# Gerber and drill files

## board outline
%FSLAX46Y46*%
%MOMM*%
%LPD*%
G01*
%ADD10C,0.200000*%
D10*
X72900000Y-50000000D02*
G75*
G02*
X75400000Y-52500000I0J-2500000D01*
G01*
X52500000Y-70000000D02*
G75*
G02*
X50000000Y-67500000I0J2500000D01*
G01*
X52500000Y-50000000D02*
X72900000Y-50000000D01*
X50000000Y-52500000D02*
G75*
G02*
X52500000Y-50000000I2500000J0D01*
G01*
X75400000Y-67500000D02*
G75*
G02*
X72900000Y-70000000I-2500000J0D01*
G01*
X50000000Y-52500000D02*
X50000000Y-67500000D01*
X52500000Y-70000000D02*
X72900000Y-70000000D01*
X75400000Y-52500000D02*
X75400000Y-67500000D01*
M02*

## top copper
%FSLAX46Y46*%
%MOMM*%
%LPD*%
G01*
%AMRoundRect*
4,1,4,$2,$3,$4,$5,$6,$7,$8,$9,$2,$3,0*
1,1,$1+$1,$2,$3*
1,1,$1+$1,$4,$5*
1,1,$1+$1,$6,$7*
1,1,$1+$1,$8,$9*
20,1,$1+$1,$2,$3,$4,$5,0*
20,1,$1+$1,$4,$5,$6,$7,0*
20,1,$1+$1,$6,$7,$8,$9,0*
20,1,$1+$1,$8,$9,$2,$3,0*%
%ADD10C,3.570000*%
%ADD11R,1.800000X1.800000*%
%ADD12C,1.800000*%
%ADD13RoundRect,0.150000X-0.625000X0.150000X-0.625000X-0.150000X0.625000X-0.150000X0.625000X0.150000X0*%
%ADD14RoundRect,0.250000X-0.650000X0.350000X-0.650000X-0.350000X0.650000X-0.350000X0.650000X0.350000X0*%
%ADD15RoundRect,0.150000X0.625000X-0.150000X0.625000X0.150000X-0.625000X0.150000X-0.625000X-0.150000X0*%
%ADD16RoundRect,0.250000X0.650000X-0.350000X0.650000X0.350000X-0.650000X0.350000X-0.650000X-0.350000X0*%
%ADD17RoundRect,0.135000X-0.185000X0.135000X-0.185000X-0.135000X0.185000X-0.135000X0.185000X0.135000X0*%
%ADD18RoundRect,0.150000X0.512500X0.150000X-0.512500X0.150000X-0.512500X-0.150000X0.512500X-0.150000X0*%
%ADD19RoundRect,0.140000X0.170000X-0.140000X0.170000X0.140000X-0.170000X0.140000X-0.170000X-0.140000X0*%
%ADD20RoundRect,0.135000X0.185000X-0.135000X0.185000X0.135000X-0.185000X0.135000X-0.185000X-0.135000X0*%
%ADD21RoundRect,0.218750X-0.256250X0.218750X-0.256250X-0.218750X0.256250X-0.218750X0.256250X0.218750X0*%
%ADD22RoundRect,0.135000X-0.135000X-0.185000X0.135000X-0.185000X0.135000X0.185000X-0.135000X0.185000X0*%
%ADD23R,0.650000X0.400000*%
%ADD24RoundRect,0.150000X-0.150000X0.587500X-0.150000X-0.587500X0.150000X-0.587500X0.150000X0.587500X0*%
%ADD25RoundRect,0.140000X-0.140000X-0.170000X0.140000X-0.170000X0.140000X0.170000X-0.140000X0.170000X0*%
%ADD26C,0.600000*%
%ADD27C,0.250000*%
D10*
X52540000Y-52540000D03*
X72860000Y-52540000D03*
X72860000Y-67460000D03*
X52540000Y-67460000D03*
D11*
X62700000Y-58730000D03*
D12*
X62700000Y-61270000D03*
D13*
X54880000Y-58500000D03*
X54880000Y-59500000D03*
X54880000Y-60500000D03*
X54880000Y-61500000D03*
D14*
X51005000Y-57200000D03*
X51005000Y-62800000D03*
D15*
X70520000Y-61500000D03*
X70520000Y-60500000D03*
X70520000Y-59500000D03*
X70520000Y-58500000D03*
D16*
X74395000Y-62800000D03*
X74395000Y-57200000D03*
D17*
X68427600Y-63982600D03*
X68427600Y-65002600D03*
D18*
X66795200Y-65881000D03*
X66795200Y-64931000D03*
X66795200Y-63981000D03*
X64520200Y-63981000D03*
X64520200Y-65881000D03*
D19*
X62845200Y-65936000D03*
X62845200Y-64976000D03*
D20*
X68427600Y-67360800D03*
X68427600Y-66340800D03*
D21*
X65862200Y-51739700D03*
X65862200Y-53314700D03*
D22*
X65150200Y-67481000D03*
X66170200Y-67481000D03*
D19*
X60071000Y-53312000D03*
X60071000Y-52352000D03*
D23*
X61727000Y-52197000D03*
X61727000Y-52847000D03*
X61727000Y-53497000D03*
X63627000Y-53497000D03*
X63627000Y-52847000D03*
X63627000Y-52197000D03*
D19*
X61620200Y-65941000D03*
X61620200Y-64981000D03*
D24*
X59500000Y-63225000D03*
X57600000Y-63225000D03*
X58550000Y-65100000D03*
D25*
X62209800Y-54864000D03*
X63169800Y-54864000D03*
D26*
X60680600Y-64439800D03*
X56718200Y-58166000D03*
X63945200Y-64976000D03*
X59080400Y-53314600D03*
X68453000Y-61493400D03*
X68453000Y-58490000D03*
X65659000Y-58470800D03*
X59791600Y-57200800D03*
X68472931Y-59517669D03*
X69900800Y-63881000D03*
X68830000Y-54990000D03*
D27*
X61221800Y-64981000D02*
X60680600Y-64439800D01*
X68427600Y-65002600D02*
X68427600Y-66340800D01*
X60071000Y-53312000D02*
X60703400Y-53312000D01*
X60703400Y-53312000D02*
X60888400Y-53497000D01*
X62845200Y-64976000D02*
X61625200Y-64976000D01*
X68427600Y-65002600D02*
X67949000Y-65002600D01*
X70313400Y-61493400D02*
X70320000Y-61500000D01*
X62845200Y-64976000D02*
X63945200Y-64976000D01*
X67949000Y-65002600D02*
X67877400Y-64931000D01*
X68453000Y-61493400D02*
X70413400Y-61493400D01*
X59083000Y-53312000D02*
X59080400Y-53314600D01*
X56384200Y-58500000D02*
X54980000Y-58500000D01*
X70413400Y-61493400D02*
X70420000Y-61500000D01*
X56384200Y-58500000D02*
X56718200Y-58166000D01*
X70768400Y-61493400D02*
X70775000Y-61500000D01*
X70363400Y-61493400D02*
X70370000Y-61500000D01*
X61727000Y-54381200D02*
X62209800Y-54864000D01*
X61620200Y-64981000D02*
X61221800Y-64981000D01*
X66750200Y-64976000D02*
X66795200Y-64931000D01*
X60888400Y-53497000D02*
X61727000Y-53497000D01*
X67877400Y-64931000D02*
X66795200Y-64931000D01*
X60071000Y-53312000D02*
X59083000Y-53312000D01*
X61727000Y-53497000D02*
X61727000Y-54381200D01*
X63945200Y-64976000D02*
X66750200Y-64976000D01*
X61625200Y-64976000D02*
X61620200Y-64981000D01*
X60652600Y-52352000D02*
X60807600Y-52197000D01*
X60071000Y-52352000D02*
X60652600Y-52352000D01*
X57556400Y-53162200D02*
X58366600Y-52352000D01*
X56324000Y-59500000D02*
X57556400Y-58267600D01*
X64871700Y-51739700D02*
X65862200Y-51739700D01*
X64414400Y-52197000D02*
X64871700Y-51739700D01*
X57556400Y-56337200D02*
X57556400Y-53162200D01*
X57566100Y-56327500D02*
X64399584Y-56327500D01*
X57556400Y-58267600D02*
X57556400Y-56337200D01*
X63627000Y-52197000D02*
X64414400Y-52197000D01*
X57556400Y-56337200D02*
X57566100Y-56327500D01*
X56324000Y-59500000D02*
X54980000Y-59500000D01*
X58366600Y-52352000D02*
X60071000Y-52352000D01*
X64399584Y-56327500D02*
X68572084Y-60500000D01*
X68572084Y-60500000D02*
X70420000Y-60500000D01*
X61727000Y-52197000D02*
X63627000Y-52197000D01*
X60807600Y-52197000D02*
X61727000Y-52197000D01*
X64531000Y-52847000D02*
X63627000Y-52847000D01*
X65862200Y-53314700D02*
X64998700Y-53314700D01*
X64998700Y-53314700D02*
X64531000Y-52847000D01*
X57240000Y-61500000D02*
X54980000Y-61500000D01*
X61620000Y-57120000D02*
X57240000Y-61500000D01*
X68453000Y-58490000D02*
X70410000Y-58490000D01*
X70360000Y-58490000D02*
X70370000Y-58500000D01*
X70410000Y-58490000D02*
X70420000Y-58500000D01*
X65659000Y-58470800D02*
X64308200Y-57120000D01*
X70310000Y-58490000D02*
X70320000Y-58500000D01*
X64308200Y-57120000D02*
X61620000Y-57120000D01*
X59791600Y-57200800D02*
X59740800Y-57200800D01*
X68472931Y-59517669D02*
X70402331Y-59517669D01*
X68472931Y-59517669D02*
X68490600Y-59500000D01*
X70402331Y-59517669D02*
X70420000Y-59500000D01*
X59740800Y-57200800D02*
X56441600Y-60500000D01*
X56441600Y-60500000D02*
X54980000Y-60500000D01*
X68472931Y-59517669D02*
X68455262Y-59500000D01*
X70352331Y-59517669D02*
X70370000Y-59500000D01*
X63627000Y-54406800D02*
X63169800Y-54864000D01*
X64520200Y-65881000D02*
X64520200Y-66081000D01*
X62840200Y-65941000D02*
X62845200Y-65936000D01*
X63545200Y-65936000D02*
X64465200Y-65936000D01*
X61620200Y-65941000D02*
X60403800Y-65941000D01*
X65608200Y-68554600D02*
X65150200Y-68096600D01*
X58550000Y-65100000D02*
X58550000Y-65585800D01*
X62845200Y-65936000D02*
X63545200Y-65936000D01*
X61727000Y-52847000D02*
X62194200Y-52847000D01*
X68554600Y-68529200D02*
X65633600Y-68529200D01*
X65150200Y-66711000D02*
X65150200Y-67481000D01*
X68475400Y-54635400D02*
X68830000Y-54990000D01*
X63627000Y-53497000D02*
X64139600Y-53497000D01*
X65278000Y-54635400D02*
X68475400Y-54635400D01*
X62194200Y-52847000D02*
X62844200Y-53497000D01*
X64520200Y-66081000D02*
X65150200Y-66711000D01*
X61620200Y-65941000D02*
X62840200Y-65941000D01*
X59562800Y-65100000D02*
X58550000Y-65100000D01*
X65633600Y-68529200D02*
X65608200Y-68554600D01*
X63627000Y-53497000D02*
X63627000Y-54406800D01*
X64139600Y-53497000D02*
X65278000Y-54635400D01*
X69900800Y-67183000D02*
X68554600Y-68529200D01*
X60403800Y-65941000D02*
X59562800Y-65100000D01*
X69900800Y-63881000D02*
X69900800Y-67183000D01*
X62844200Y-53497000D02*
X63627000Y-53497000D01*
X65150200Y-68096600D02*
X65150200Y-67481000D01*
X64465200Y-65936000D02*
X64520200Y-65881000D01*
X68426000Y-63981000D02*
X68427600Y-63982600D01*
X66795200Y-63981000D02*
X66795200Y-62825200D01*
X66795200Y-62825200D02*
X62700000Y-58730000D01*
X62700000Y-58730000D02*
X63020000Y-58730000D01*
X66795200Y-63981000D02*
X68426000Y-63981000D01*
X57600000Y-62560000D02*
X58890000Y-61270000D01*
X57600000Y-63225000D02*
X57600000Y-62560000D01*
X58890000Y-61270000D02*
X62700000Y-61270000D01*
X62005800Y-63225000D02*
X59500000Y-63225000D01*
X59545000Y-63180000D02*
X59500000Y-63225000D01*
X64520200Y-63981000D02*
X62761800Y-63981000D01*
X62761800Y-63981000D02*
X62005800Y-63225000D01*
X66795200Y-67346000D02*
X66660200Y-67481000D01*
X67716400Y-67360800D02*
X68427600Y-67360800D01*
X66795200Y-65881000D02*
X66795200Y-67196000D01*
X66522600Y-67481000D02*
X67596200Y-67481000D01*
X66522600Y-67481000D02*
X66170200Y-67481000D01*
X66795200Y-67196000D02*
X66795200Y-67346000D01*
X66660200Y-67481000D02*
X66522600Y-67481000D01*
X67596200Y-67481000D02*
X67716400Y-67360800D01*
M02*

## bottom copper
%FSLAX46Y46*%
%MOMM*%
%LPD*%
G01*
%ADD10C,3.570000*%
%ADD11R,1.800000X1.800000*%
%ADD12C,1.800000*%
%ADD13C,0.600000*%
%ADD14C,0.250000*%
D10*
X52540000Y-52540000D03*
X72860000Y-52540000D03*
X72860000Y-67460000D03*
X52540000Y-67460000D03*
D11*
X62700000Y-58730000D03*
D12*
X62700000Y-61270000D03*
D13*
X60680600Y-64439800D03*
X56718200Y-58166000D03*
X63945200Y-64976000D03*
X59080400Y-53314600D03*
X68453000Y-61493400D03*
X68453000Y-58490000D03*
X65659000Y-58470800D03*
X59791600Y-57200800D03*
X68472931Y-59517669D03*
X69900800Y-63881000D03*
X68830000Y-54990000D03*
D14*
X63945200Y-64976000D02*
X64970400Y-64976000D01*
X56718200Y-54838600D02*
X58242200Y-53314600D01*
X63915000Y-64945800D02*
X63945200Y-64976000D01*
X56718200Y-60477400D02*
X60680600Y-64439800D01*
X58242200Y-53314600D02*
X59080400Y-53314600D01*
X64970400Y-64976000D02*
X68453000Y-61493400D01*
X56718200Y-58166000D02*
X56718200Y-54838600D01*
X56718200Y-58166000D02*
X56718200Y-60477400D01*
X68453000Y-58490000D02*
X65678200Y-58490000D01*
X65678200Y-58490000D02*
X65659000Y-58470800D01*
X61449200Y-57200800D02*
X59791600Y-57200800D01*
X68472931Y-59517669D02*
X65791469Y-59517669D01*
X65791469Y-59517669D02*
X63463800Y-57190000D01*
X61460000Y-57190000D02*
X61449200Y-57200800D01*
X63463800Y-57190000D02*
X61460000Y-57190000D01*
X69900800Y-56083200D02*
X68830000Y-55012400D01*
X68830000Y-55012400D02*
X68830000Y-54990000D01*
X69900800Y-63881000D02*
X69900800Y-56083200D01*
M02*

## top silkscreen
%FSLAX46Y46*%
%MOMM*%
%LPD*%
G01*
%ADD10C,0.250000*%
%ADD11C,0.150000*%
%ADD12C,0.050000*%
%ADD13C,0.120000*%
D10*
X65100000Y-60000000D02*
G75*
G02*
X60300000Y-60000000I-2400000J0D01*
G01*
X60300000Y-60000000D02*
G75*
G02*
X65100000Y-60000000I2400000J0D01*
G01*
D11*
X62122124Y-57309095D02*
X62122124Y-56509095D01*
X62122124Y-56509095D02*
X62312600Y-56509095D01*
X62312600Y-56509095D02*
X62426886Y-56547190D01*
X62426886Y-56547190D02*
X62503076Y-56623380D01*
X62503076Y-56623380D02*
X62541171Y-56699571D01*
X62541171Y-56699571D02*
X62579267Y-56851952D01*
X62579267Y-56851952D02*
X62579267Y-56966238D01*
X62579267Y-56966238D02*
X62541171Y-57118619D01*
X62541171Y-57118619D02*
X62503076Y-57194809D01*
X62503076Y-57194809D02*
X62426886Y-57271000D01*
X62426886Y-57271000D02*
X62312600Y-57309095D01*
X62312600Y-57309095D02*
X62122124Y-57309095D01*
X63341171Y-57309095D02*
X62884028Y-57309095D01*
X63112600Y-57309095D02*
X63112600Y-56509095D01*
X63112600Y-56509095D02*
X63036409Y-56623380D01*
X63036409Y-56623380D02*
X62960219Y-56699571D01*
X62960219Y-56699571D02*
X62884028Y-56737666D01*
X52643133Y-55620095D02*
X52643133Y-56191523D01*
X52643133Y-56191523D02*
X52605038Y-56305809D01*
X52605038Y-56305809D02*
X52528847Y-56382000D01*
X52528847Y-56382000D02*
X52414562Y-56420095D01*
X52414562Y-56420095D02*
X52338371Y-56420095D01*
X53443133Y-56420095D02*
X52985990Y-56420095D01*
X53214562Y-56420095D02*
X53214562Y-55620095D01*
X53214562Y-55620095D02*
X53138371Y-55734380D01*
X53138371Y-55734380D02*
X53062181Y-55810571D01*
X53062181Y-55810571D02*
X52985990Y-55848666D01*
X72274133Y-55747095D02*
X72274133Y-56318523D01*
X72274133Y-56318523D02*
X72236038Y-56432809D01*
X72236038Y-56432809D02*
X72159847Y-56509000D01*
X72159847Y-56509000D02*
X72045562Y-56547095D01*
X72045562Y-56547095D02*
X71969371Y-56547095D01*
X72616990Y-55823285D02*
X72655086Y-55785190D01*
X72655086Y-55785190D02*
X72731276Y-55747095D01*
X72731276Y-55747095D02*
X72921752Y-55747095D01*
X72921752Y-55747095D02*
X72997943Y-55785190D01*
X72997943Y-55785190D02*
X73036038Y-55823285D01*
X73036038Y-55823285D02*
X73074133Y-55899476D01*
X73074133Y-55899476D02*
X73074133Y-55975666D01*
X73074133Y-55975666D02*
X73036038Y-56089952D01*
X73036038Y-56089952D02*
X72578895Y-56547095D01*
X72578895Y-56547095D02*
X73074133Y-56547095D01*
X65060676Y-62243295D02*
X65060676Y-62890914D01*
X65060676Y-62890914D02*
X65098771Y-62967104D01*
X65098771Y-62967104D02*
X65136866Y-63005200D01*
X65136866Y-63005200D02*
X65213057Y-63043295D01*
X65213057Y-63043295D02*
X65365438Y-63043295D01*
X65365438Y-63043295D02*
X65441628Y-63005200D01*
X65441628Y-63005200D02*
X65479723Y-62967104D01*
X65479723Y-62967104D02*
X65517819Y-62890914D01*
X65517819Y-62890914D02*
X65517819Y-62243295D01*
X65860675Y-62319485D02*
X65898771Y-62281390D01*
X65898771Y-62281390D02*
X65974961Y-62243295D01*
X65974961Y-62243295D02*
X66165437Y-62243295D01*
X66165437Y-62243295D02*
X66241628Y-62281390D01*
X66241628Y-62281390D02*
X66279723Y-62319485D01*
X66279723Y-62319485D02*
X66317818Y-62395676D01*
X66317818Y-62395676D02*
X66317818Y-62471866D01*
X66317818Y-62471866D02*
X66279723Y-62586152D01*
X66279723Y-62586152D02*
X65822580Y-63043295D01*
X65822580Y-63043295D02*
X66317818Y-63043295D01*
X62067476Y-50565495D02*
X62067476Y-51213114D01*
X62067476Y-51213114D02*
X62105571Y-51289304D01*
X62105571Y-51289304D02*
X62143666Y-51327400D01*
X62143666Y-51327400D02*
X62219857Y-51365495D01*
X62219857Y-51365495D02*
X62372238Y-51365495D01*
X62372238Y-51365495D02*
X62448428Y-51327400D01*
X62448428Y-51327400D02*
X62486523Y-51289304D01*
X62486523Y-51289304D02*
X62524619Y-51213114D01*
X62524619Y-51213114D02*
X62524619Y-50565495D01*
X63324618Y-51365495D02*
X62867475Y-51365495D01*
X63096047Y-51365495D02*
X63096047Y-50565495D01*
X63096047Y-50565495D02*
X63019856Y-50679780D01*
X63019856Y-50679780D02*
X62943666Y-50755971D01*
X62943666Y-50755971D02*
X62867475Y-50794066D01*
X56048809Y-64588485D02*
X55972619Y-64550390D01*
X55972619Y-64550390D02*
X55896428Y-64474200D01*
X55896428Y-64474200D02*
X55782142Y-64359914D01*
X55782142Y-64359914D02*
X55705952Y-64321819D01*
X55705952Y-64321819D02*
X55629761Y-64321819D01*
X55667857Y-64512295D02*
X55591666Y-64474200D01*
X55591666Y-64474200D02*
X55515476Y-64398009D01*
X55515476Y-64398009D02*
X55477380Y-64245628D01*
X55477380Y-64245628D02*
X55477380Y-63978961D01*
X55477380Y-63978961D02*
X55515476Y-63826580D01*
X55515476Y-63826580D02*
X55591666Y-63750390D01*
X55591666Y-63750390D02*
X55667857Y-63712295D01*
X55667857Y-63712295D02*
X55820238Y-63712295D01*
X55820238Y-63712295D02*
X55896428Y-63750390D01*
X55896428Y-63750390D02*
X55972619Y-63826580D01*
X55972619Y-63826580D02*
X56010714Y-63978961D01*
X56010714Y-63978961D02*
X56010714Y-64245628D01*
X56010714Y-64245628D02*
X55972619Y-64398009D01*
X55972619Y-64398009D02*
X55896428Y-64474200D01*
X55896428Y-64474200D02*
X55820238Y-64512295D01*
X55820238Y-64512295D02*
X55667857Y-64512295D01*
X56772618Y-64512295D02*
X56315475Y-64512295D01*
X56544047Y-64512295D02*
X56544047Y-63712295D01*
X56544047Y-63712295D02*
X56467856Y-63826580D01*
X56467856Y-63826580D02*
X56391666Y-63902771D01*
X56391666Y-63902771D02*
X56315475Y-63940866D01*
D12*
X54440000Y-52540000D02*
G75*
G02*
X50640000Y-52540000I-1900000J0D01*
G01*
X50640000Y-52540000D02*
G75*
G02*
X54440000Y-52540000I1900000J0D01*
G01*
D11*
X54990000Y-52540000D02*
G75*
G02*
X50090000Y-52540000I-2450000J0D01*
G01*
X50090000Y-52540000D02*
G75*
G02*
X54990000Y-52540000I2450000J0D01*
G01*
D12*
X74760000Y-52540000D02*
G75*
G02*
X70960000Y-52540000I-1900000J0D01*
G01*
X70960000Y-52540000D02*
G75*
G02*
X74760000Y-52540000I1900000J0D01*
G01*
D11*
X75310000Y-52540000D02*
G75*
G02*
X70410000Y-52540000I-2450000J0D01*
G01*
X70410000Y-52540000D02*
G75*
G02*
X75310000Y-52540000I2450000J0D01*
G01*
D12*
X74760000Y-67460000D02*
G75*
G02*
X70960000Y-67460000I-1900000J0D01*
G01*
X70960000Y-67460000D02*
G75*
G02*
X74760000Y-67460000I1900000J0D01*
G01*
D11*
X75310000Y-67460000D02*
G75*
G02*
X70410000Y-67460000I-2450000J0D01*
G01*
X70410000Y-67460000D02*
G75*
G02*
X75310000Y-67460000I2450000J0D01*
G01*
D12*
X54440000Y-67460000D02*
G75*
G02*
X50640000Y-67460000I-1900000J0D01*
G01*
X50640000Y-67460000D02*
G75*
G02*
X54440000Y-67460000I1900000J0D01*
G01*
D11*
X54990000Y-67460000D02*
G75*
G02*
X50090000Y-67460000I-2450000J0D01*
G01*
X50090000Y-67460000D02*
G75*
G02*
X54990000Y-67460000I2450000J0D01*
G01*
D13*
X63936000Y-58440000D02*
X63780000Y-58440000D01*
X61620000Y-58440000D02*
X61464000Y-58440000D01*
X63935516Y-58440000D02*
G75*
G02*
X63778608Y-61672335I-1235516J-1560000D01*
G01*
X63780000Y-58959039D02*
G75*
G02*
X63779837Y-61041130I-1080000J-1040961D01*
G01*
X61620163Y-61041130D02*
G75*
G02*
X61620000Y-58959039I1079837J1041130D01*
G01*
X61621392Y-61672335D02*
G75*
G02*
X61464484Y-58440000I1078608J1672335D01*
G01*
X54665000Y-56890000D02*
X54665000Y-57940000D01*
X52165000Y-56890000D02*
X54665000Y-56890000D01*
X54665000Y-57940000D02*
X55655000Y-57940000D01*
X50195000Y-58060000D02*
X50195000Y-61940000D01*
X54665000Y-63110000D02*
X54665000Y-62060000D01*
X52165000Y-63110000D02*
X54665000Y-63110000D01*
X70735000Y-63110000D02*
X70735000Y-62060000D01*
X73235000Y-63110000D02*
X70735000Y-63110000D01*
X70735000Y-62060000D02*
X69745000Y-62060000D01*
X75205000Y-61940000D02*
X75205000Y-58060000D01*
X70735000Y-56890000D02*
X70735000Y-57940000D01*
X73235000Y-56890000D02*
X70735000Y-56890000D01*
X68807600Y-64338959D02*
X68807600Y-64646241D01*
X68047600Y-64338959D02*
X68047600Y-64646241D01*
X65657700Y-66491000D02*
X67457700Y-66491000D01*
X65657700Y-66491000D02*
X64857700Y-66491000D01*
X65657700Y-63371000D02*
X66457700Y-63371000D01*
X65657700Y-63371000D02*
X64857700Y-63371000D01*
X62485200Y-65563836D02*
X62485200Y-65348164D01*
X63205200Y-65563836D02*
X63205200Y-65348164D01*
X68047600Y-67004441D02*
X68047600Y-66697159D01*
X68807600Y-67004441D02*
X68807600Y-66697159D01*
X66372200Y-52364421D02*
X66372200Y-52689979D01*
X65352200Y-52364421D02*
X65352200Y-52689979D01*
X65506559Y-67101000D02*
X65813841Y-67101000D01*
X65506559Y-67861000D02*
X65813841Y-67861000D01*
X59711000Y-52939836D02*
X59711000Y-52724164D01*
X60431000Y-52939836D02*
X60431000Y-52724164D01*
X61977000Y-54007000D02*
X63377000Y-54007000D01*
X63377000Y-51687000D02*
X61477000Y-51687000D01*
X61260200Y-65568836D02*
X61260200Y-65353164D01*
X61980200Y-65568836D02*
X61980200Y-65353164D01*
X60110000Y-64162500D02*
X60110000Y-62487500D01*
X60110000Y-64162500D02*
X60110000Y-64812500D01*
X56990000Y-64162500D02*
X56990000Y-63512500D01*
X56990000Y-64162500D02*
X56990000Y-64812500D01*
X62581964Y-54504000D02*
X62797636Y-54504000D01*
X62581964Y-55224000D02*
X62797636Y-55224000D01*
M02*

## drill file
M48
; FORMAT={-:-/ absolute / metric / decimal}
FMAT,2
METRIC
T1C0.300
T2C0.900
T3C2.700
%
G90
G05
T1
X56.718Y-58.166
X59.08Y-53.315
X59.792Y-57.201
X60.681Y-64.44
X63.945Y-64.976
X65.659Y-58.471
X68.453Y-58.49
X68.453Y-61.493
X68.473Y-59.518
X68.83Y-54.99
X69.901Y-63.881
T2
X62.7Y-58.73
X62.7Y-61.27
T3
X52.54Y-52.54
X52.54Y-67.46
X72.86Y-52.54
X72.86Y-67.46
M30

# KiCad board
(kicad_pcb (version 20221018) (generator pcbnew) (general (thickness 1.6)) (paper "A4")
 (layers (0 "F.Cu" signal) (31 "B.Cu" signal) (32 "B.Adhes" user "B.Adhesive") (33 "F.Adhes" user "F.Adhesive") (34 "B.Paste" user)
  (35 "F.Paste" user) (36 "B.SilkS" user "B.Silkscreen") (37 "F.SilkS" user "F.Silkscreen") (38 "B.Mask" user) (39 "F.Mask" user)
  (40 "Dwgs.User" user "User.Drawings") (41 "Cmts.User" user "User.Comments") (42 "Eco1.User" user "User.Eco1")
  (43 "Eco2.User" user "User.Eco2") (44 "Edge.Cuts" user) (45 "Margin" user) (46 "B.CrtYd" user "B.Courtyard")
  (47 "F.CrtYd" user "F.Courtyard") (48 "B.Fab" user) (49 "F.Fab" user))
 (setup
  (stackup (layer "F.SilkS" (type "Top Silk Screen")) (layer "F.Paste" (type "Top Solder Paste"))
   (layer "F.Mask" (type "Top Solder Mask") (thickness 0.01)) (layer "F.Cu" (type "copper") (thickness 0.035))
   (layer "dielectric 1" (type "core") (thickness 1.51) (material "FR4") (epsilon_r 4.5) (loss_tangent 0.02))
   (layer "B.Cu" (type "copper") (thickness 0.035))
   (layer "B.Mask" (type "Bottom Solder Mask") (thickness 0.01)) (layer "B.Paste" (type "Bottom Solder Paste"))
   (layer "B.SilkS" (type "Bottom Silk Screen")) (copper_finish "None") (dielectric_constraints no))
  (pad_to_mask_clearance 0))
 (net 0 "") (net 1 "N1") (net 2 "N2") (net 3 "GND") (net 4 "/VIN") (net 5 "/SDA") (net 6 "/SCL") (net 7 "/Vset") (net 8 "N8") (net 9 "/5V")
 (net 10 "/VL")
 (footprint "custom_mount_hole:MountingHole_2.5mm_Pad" (layer "F.Cu") (at 52.54 52.54)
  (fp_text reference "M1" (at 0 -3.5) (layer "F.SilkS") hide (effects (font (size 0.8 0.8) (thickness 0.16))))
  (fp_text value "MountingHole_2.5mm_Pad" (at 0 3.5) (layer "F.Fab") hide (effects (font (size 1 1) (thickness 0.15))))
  (fp_circle (center 0 0) (end 1.9 0) (stroke (width 0.05) (type solid)) (fill none) (layer "F.SilkS"))
  (fp_circle (center 0 0) (end 2.45 0) (stroke (width 0.15) (type solid)) (fill none) (layer "F.SilkS"))
  (pad "~" thru_hole circle (at 0 0) (size 3.57 3.57) (drill 2.7) (layers "*.Cu" "*.Mask")))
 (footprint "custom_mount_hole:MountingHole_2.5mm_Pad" (layer "F.Cu") (at 72.86 52.54)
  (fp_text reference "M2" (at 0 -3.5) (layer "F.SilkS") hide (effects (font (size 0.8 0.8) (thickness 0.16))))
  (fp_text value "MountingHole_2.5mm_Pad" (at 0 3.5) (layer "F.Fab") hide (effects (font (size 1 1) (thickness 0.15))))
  (fp_circle (center 0 0) (end 1.9 0) (stroke (width 0.05) (type solid)) (fill none) (layer "F.SilkS"))
  (fp_circle (center 0 0) (end 2.45 0) (stroke (width 0.15) (type solid)) (fill none) (layer "F.SilkS"))
  (pad "~" thru_hole circle (at 0 0) (size 3.57 3.57) (drill 2.7) (layers "*.Cu" "*.Mask")))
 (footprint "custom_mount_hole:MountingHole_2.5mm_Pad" (layer "F.Cu") (at 72.86 67.46)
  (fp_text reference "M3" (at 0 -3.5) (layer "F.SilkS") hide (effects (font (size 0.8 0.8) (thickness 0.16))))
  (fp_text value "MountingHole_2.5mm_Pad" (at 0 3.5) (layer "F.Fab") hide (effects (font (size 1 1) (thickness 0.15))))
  (fp_circle (center 0 0) (end 1.9 0) (stroke (width 0.05) (type solid)) (fill none) (layer "F.SilkS"))
  (fp_circle (center 0 0) (end 2.45 0) (stroke (width 0.15) (type solid)) (fill none) (layer "F.SilkS"))
  (pad "~" thru_hole circle (at 0 0) (size 3.57 3.57) (drill 2.7) (layers "*.Cu" "*.Mask")))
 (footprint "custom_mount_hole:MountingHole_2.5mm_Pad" (layer "F.Cu") (at 52.54 67.46)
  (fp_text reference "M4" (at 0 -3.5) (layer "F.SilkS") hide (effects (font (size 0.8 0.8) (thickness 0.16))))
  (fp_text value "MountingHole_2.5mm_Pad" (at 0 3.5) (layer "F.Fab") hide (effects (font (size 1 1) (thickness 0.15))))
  (fp_circle (center 0 0) (end 1.9 0) (stroke (width 0.05) (type solid)) (fill none) (layer "F.SilkS"))
  (fp_circle (center 0 0) (end 2.45 0) (stroke (width 0.15) (type solid)) (fill none) (layer "F.SilkS"))
  (pad "~" thru_hole circle (at 0 0) (size 3.57 3.57) (drill 2.7) (layers "*.Cu" "*.Mask")))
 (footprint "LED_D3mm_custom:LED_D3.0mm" (layer "F.Cu") (at 62.7 58.73 -90)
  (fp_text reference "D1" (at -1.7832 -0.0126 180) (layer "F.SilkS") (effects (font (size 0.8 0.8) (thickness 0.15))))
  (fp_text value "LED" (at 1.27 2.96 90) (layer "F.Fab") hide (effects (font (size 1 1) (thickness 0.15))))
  (fp_line (start -0.29 -1.236) (end -0.29 -1.08) (stroke (width 0.12) (type solid)) (layer "F.SilkS"))
  (fp_line (start -0.29 1.08) (end -0.29 1.236) (stroke (width 0.12) (type solid)) (layer "F.SilkS"))
  (fp_arc (start -0.29 -1.235516) (mid 1.366487 -1.987659) (end 2.942335 -1.078608) (stroke (width 0.12) (type solid)) (layer "F.SilkS"))
  (fp_arc (start 0.229039 -1.08) (mid 1.270117 -1.5) (end 2.31113 -1.079837) (stroke (width 0.12) (type solid)) (layer "F.SilkS"))
  (fp_arc (start 2.31113 1.079837) (mid 1.270117 1.5) (end 0.229039 1.08) (stroke (width 0.12) (type solid)) (layer "F.SilkS"))
  (fp_arc (start 2.942335 1.078608) (mid 1.366487 1.987659) (end -0.29 1.235516) (stroke (width 0.12) (type solid)) (layer "F.SilkS"))
  (pad "1" thru_hole rect (at 0 0 270) (size 1.8 1.8) (drill 0.9) (layers "*.Cu" "*.Mask") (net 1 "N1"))
  (pad "2" thru_hole circle (at 2.54 0 270) (size 1.8 1.8) (drill 0.9) (layers "*.Cu" "*.Mask") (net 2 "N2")))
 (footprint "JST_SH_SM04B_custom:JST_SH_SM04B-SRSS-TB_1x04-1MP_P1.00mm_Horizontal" (layer "F.Cu") (at 52.88 60 -90)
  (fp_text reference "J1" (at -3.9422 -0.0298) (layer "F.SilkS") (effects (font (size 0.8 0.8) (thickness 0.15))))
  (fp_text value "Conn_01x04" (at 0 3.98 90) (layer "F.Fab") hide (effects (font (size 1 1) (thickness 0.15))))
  (fp_line (start -3.11 -1.785) (end -2.06 -1.785) (stroke (width 0.12) (type solid)) (layer "F.SilkS"))
  (fp_line (start -3.11 0.715) (end -3.11 -1.785) (stroke (width 0.12) (type solid)) (layer "F.SilkS"))
  (fp_line (start -2.06 -1.785) (end -2.06 -2.775) (stroke (width 0.12) (type solid)) (layer "F.SilkS"))
  (fp_line (start -1.94 2.685) (end 1.94 2.685) (stroke (width 0.12) (type solid)) (layer "F.SilkS"))
  (fp_line (start 3.11 -1.785) (end 2.06 -1.785) (stroke (width 0.12) (type solid)) (layer "F.SilkS"))
  (fp_line (start 3.11 0.715) (end 3.11 -1.785) (stroke (width 0.12) (type solid)) (layer "F.SilkS"))
  (pad "1" smd roundrect (at -1.5 -2 270) (size 0.6 1.55) (layers "F.Cu" "F.Paste" "F.Mask") (roundrect_rratio 0.25) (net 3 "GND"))
  (pad "2" smd roundrect (at -0.5 -2 270) (size 0.6 1.55) (layers "F.Cu" "F.Paste" "F.Mask") (roundrect_rratio 0.25) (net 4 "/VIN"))
  (pad "3" smd roundrect (at 0.5 -2 270) (size 0.6 1.55) (layers "F.Cu" "F.Paste" "F.Mask") (roundrect_rratio 0.25) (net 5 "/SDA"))
  (pad "4" smd roundrect (at 1.5 -2 270) (size 0.6 1.55) (layers "F.Cu" "F.Paste" "F.Mask") (roundrect_rratio 0.25) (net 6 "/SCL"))
  (pad "MP" smd roundrect (at -2.8 1.875 270) (size 1.2 1.8) (layers "F.Cu" "F.Paste" "F.Mask") (roundrect_rratio 0.2083333333))
  (pad "MP" smd roundrect (at 2.8 1.875 270) (size 1.2 1.8) (layers "F.Cu" "F.Paste" "F.Mask") (roundrect_rratio 0.2083333333)))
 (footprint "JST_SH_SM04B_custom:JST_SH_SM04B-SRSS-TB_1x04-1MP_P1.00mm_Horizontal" (layer "F.Cu") (at 72.52 60 90)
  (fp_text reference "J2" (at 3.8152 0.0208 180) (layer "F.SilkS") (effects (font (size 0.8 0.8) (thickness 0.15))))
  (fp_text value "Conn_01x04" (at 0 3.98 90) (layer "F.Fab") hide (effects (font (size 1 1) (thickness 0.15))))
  (fp_line (start -3.11 -1.785) (end -2.06 -1.785) (stroke (width 0.12) (type solid)) (layer "F.SilkS"))
  (fp_line (start -3.11 0.715) (end -3.11 -1.785) (stroke (width 0.12) (type solid)) (layer "F.SilkS"))
  (fp_line (start -2.06 -1.785) (end -2.06 -2.775) (stroke (width 0.12) (type solid)) (layer "F.SilkS"))
  (fp_line (start -1.94 2.685) (end 1.94 2.685) (stroke (width 0.12) (type solid)) (layer "F.SilkS"))
  (fp_line (start 3.11 -1.785) (end 2.06 -1.785) (stroke (width 0.12) (type solid)) (layer "F.SilkS"))
  (fp_line (start 3.11 0.715) (end 3.11 -1.785) (stroke (width 0.12) (type solid)) (layer "F.SilkS"))
  (pad "1" smd roundrect (at -1.5 -2 90) (size 0.6 1.55) (layers "F.Cu" "F.Paste" "F.Mask") (roundrect_rratio 0.25) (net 3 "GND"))
  (pad "2" smd roundrect (at -0.5 -2 90) (size 0.6 1.55) (layers "F.Cu" "F.Paste" "F.Mask") (roundrect_rratio 0.25) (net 4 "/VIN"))
  (pad "3" smd roundrect (at 0.5 -2 90) (size 0.6 1.55) (layers "F.Cu" "F.Paste" "F.Mask") (roundrect_rratio 0.25) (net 5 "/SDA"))
  (pad "4" smd roundrect (at 1.5 -2 90) (size 0.6 1.55) (layers "F.Cu" "F.Paste" "F.Mask") (roundrect_rratio 0.25) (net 6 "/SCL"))
  (pad "MP" smd roundrect (at -2.8 1.875 90) (size 1.2 1.8) (layers "F.Cu" "F.Paste" "F.Mask") (roundrect_rratio 0.2083333333))
  (pad "MP" smd roundrect (at 2.8 1.875 90) (size 1.2 1.8) (layers "F.Cu" "F.Paste" "F.Mask") (roundrect_rratio 0.2083333333)))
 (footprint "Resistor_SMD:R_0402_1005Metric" (layer "F.Cu") (at 68.4276 64.4926 -90)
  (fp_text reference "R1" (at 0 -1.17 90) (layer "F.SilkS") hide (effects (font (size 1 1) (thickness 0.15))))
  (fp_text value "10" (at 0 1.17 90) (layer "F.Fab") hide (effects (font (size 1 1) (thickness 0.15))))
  (fp_line (start -0.153641 -0.38) (end 0.153641 -0.38) (stroke (width 0.12) (type solid)) (layer "F.SilkS"))
  (fp_line (start -0.153641 0.38) (end 0.153641 0.38) (stroke (width 0.12) (type solid)) (layer "F.SilkS"))
  (pad "1" smd roundrect (at -0.51 0 270) (size 0.54 0.64) (layers "F.Cu" "F.Paste" "F.Mask") (roundrect_rratio 0.25) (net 1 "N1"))
  (pad "2" smd roundrect (at 0.51 0 270) (size 0.54 0.64) (layers "F.Cu" "F.Paste" "F.Mask") (roundrect_rratio 0.25) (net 3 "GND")))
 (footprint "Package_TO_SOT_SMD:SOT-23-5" (layer "F.Cu") (at 65.6577 64.931 180)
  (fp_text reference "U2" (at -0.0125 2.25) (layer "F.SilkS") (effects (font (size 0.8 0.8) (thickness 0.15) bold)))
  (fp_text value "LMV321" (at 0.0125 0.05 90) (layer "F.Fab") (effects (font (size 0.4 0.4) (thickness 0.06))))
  (fp_line (start 0 -1.56) (end -1.8 -1.56) (stroke (width 0.12) (type solid)) (layer "F.SilkS"))
  (fp_line (start 0 -1.56) (end 0.8 -1.56) (stroke (width 0.12) (type solid)) (layer "F.SilkS"))
  (fp_line (start 0 1.56) (end -0.8 1.56) (stroke (width 0.12) (type solid)) (layer "F.SilkS"))
  (fp_line (start 0 1.56) (end 0.8 1.56) (stroke (width 0.12) (type solid)) (layer "F.SilkS"))
  (pad "1" smd roundrect (at -1.1375 -0.95 180) (size 1.325 0.6) (layers "F.Cu" "F.Paste" "F.Mask") (roundrect_rratio 0.25) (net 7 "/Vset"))
  (pad "2" smd roundrect (at -1.1375 0 180) (size 1.325 0.6) (layers "F.Cu" "F.Paste" "F.Mask") (roundrect_rratio 0.25) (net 3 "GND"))
  (pad "3" smd roundrect (at -1.1375 0.95 180) (size 1.325 0.6) (layers "F.Cu" "F.Paste" "F.Mask") (roundrect_rratio 0.25) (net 1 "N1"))
  (pad "4" smd roundrect (at 1.1375 0.95 180) (size 1.325 0.6) (layers "F.Cu" "F.Paste" "F.Mask") (roundrect_rratio 0.25) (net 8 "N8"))
  (pad "5" smd roundrect (at 1.1375 -0.95 180) (size 1.325 0.6) (layers "F.Cu" "F.Paste" "F.Mask") (roundrect_rratio 0.25) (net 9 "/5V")))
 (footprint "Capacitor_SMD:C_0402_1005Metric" (layer "F.Cu") (at 62.8452 65.456 90)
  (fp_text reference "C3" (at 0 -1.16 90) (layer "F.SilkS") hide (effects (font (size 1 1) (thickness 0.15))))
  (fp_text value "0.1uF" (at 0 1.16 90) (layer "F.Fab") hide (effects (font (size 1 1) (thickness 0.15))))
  (fp_line (start -0.107836 -0.36) (end 0.107836 -0.36) (stroke (width 0.12) (type solid)) (layer "F.SilkS"))
  (fp_line (start -0.107836 0.36) (end 0.107836 0.36) (stroke (width 0.12) (type solid)) (layer "F.SilkS"))
  (pad "1" smd roundrect (at -0.48 0 90) (size 0.56 0.62) (layers "F.Cu" "F.Paste" "F.Mask") (roundrect_rratio 0.25) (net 9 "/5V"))
  (pad "2" smd roundrect (at 0.48 0 90) (size 0.56 0.62) (layers "F.Cu" "F.Paste" "F.Mask") (roundrect_rratio 0.25) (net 3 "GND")))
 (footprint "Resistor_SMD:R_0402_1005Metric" (layer "F.Cu") (at 68.4276 66.8508 90)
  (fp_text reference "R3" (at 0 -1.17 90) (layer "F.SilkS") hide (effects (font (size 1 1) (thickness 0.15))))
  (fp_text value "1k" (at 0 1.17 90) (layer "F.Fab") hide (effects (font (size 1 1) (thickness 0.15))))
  (fp_line (start -0.153641 -0.38) (end 0.153641 -0.38) (stroke (width 0.12) (type solid)) (layer "F.SilkS"))
  (fp_line (start -0.153641 0.38) (end 0.153641 0.38) (stroke (width 0.12) (type solid)) (layer "F.SilkS"))
  (pad "1" smd roundrect (at -0.51 0 90) (size 0.54 0.64) (layers "F.Cu" "F.Paste" "F.Mask") (roundrect_rratio 0.25) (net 7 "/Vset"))
  (pad "2" smd roundrect (at 0.51 0 90) (size 0.54 0.64) (layers "F.Cu" "F.Paste" "F.Mask") (roundrect_rratio 0.25) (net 3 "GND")))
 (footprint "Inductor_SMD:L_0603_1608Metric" (layer "F.Cu") (at 65.8622 52.5272 -90)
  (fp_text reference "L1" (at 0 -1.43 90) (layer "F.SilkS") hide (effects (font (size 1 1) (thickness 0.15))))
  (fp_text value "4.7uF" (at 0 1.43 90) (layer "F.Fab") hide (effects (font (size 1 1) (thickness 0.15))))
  (fp_line (start -0.162779 -0.51) (end 0.162779 -0.51) (stroke (width 0.12) (type solid)) (layer "F.SilkS"))
  (fp_line (start -0.162779 0.51) (end 0.162779 0.51) (stroke (width 0.12) (type solid)) (layer "F.SilkS"))
  (pad "1" smd roundrect (at -0.7875 0 270) (size 0.875 0.95) (layers "F.Cu" "F.Paste" "F.Mask") (roundrect_rratio 0.25) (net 4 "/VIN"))
  (pad "2" smd roundrect (at 0.7875 0 270) (size 0.875 0.95) (layers "F.Cu" "F.Paste" "F.Mask") (roundrect_rratio 0.25) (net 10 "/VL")))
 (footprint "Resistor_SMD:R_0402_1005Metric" (layer "F.Cu") (at 65.6602 67.481)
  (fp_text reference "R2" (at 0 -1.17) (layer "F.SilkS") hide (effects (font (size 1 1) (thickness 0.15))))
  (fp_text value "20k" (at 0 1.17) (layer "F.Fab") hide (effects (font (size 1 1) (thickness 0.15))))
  (fp_line (start -0.153641 -0.38) (end 0.153641 -0.38) (stroke (width 0.12) (type solid)) (layer "F.SilkS"))
  (fp_line (start -0.153641 0.38) (end 0.153641 0.38) (stroke (width 0.12) (type solid)) (layer "F.SilkS"))
  (pad "1" smd roundrect (at -0.51 0) (size 0.54 0.64) (layers "F.Cu" "F.Paste" "F.Mask") (roundrect_rratio 0.25) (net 9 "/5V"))
  (pad "2" smd roundrect (at 0.51 0) (size 0.54 0.64) (layers "F.Cu" "F.Paste" "F.Mask") (roundrect_rratio 0.25) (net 7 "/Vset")))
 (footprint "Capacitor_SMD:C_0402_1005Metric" (layer "F.Cu") (at 60.071 52.832 90)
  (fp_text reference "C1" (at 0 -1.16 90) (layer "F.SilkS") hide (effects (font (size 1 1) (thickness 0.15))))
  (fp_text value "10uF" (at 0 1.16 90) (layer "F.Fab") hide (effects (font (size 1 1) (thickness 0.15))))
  (fp_line (start -0.107836 -0.36) (end 0.107836 -0.36) (stroke (width 0.12) (type solid)) (layer "F.SilkS"))
  (fp_line (start -0.107836 0.36) (end 0.107836 0.36) (stroke (width 0.12) (type solid)) (layer "F.SilkS"))
  (pad "1" smd roundrect (at -0.48 0 90) (size 0.56 0.62) (layers "F.Cu" "F.Paste" "F.Mask") (roundrect_rratio 0.25) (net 3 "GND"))
  (pad "2" smd roundrect (at 0.48 0 90) (size 0.56 0.62) (layers "F.Cu" "F.Paste" "F.Mask") (roundrect_rratio 0.25) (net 4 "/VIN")))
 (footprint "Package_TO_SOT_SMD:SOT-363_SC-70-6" (layer "F.Cu") (at 62.677 52.847)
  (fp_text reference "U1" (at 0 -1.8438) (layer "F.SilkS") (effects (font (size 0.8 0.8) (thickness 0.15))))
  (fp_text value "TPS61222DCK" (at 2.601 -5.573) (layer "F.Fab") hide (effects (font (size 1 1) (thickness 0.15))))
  (fp_line (start -0.7 1.16) (end 0.7 1.16) (stroke (width 0.12) (type solid)) (layer "F.SilkS"))
  (fp_line (start 0.7 -1.16) (end -1.2 -1.16) (stroke (width 0.12) (type solid)) (layer "F.SilkS"))
  (pad "1" smd rect (at -0.95 -0.65) (size 0.65 0.4) (layers "F.Cu" "F.Paste" "F.Mask") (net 4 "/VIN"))
  (pad "2" smd rect (at -0.95 0) (size 0.65 0.4) (layers "F.Cu" "F.Paste" "F.Mask") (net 9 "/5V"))
  (pad "3" smd rect (at -0.95 0.65) (size 0.65 0.4) (layers "F.Cu" "F.Paste" "F.Mask") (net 3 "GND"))
  (pad "4" smd rect (at 0.95 0.65) (size 0.65 0.4) (layers "F.Cu" "F.Paste" "F.Mask") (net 9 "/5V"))
  (pad "5" smd rect (at 0.95 0) (size 0.65 0.4) (layers "F.Cu" "F.Paste" "F.Mask") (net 10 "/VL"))
  (pad "6" smd rect (at 0.95 -0.65) (size 0.65 0.4) (layers "F.Cu" "F.Paste" "F.Mask") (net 4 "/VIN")))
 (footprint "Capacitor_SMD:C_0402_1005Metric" (layer "F.Cu") (at 61.6202 65.461 90)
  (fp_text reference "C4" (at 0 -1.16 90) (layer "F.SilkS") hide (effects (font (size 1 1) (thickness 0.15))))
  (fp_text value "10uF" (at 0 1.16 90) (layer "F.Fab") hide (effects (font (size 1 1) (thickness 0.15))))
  (fp_line (start -0.107836 -0.36) (end 0.107836 -0.36) (stroke (width 0.12) (type solid)) (layer "F.SilkS"))
  (fp_line (start -0.107836 0.36) (end 0.107836 0.36) (stroke (width 0.12) (type solid)) (layer "F.SilkS"))
  (pad "1" smd roundrect (at -0.48 0 90) (size 0.56 0.62) (layers "F.Cu" "F.Paste" "F.Mask") (roundrect_rratio 0.25) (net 9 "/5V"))
  (pad "2" smd roundrect (at 0.48 0 90) (size 0.56 0.62) (layers "F.Cu" "F.Paste" "F.Mask") (roundrect_rratio 0.25) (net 3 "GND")))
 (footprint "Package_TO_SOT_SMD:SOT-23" (layer "F.Cu") (at 58.55 64.1625 -90)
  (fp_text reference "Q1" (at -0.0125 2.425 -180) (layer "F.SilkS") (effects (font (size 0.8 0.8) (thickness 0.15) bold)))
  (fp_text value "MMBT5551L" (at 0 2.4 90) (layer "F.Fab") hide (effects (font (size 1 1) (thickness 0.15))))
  (fp_line (start 0 -1.56) (end -1.675 -1.56) (stroke (width 0.12) (type solid)) (layer "F.SilkS"))
  (fp_line (start 0 -1.56) (end 0.65 -1.56) (stroke (width 0.12) (type solid)) (layer "F.SilkS"))
  (fp_line (start 0 1.56) (end -0.65 1.56) (stroke (width 0.12) (type solid)) (layer "F.SilkS"))
  (fp_line (start 0 1.56) (end 0.65 1.56) (stroke (width 0.12) (type solid)) (layer "F.SilkS"))
  (pad "1" smd roundrect (at -0.9375 -0.95 270) (size 1.475 0.6) (layers "F.Cu" "F.Paste" "F.Mask") (roundrect_rratio 0.25) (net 8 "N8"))
  (pad "2" smd roundrect (at -0.9375 0.95 270) (size 1.475 0.6) (layers "F.Cu" "F.Paste" "F.Mask") (roundrect_rratio 0.25) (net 2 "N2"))
  (pad "3" smd roundrect (at 0.9375 0 270) (size 1.475 0.6) (layers "F.Cu" "F.Paste" "F.Mask") (roundrect_rratio 0.25) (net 9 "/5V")))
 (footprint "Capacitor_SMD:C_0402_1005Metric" (layer "F.Cu") (at 62.6898 54.864)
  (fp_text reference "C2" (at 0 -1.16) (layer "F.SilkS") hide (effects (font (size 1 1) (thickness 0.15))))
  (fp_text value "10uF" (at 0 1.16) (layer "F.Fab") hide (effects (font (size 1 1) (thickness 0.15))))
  (fp_line (start -0.107836 -0.36) (end 0.107836 -0.36) (stroke (width 0.12) (type solid)) (layer "F.SilkS"))
  (fp_line (start -0.107836 0.36) (end 0.107836 0.36) (stroke (width 0.12) (type solid)) (layer "F.SilkS"))
  (pad "1" smd roundrect (at -0.48 0) (size 0.56 0.62) (layers "F.Cu" "F.Paste" "F.Mask") (roundrect_rratio 0.25) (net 3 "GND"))
  (pad "2" smd roundrect (at 0.48 0) (size 0.56 0.62) (layers "F.Cu" "F.Paste" "F.Mask") (roundrect_rratio 0.25) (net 9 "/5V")))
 (gr_circle (center 62.7 60) (end 65.1 60) (stroke (width 0.25) (type solid)) (fill none) (layer "F.SilkS"))
 (gr_arc (start 72.9 50) (mid 74.667767 50.732233) (end 75.4 52.5) (stroke (width 0.2) (type solid)) (layer "Edge.Cuts"))
 (gr_arc (start 52.5 70) (mid 50.732233 69.267767) (end 50 67.5) (stroke (width 0.2) (type solid)) (layer "Edge.Cuts"))
 (gr_line (start 52.5 50) (end 72.9 50) (stroke (width 0.2) (type solid)) (layer "Edge.Cuts"))
 (gr_arc (start 50 52.5) (mid 50.732233 50.732233) (end 52.5 50) (stroke (width 0.2) (type solid)) (layer "Edge.Cuts"))
 (gr_arc (start 75.4 67.5) (mid 74.667767 69.267767) (end 72.9 70) (stroke (width 0.2) (type solid)) (layer "Edge.Cuts"))
 (gr_line (start 50 52.5) (end 50 67.5) (stroke (width 0.2) (type solid)) (layer "Edge.Cuts"))
 (gr_line (start 52.5 70) (end 72.9 70) (stroke (width 0.2) (type solid)) (layer "Edge.Cuts"))
 (gr_line (start 75.4 52.5) (end 75.4 67.5) (stroke (width 0.2) (type solid)) (layer "Edge.Cuts"))
 (segment (start 61.2218 64.981) (end 60.6806 64.4398) (width 0.25) (layer "F.Cu") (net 3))
 (segment (start 68.4276 65.0026) (end 68.4276 66.3408) (width 0.25) (layer "F.Cu") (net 3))
 (segment (start 60.071 53.312) (end 60.7034 53.312) (width 0.25) (layer "F.Cu") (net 3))
 (segment (start 60.7034 53.312) (end 60.8884 53.497) (width 0.25) (layer "F.Cu") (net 3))
 (segment (start 62.8452 64.976) (end 61.6252 64.976) (width 0.25) (layer "F.Cu") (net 3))
 (segment (start 68.4276 65.0026) (end 67.949 65.0026) (width 0.25) (layer "F.Cu") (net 3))
 (segment (start 70.3134 61.4934) (end 70.32 61.5) (width 0.25) (layer "F.Cu") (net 3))
 (segment (start 62.8452 64.976) (end 63.9452 64.976) (width 0.25) (layer "F.Cu") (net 3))
 (segment (start 67.949 65.0026) (end 67.8774 64.931) (width 0.25) (layer "F.Cu") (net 3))
 (segment (start 68.453 61.4934) (end 70.4134 61.4934) (width 0.25) (layer "F.Cu") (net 3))
 (segment (start 59.083 53.312) (end 59.0804 53.3146) (width 0.25) (layer "F.Cu") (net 3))
 (segment (start 56.3842 58.5) (end 54.98 58.5) (width 0.25) (layer "F.Cu") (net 3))
 (segment (start 70.4134 61.4934) (end 70.42 61.5) (width 0.25) (layer "F.Cu") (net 3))
 (segment (start 56.3842 58.5) (end 56.7182 58.166) (width 0.25) (layer "F.Cu") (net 3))
 (segment (start 70.7684 61.4934) (end 70.775 61.5) (width 0.25) (layer "F.Cu") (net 3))
 (segment (start 70.3634 61.4934) (end 70.37 61.5) (width 0.25) (layer "F.Cu") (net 3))
 (segment (start 61.727 54.3812) (end 62.2098 54.864) (width 0.25) (layer "F.Cu") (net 3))
 (segment (start 61.6202 64.981) (end 61.2218 64.981) (width 0.25) (layer "F.Cu") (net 3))
 (segment (start 66.7502 64.976) (end 66.7952 64.931) (width 0.25) (layer "F.Cu") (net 3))
 (segment (start 60.8884 53.497) (end 61.727 53.497) (width 0.25) (layer "F.Cu") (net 3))
 (segment (start 67.8774 64.931) (end 66.7952 64.931) (width 0.25) (layer "F.Cu") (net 3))
 (segment (start 60.071 53.312) (end 59.083 53.312) (width 0.25) (layer "F.Cu") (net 3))
 (segment (start 61.727 53.497) (end 61.727 54.3812) (width 0.25) (layer "F.Cu") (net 3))
 (segment (start 63.9452 64.976) (end 66.7502 64.976) (width 0.25) (layer "F.Cu") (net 3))
 (segment (start 61.6252 64.976) (end 61.6202 64.981) (width 0.25) (layer "F.Cu") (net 3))
 (via (at 60.6806 64.4398) (size 0.6) (drill 0.3) (layers "F.Cu" "B.Cu") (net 3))
 (via (at 56.7182 58.166) (size 0.6) (drill 0.3) (layers "F.Cu" "B.Cu") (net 3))
 (via (at 63.9452 64.976) (size 0.6) (drill 0.3) (layers "F.Cu" "B.Cu") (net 3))
 (via (at 59.0804 53.3146) (size 0.6) (drill 0.3) (layers "F.Cu" "B.Cu") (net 3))
 (via (at 68.453 61.4934) (size 0.6) (drill 0.3) (layers "F.Cu" "B.Cu") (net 3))
 (segment (start 63.9452 64.976) (end 64.9704 64.976) (width 0.25) (layer "B.Cu") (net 3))
 (segment (start 56.7182 54.8386) (end 58.2422 53.3146) (width 0.25) (layer "B.Cu") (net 3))
 (segment (start 63.915 64.9458) (end 63.9452 64.976) (width 0.25) (layer "B.Cu") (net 3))
 (segment (start 56.7182 60.4774) (end 60.6806 64.4398) (width 0.25) (layer "B.Cu") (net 3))
 (segment (start 58.2422 53.3146) (end 59.0804 53.3146) (width 0.25) (layer "B.Cu") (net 3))
 (segment (start 64.9704 64.976) (end 68.453 61.4934) (width 0.25) (layer "B.Cu") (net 3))
 (segment (start 56.7182 58.166) (end 56.7182 54.8386) (width 0.25) (layer "B.Cu") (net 3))
 (segment (start 56.7182 58.166) (end 56.7182 60.4774) (width 0.25) (layer "B.Cu") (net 3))
 (segment (start 60.6526 52.352) (end 60.8076 52.197) (width 0.25) (layer "F.Cu") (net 4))
 (segment (start 60.071 52.352) (end 60.6526 52.352) (width 0.25) (layer "F.Cu") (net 4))
 (segment (start 57.5564 53.1622) (end 58.3666 52.352) (width 0.25) (layer "F.Cu") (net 4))
 (segment (start 56.324 59.5) (end 57.5564 58.2676) (width 0.25) (layer "F.Cu") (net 4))
 (segment (start 64.8717 51.7397) (end 65.8622 51.7397) (width 0.25) (layer "F.Cu") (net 4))
 (segment (start 64.4144 52.197) (end 64.8717 51.7397) (width 0.25) (layer "F.Cu") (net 4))
 (segment (start 57.5564 56.3372) (end 57.5564 53.1622) (width 0.25) (layer "F.Cu") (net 4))
 (segment (start 57.5661 56.3275) (end 64.399584 56.3275) (width 0.25) (layer "F.Cu") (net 4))
 (segment (start 57.5564 58.2676) (end 57.5564 56.3372) (width 0.25) (layer "F.Cu") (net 4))
 (segment (start 63.627 52.197) (end 64.4144 52.197) (width 0.25) (layer "F.Cu") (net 4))
 (segment (start 57.5564 56.3372) (end 57.5661 56.3275) (width 0.25) (layer "F.Cu") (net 4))
 (segment (start 56.324 59.5) (end 54.98 59.5) (width 0.25) (layer "F.Cu") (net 4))
 (segment (start 58.3666 52.352) (end 60.071 52.352) (width 0.25) (layer "F.Cu") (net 4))
 (segment (start 64.399584 56.3275) (end 68.572084 60.5) (width 0.25) (layer "F.Cu") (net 4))
 (segment (start 68.572084 60.5) (end 70.42 60.5) (width 0.25) (layer "F.Cu") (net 4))
 (segment (start 61.727 52.197) (end 63.627 52.197) (width 0.25) (layer "F.Cu") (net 4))
 (segment (start 60.8076 52.197) (end 61.727 52.197) (width 0.25) (layer "F.Cu") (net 4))
 (segment (start 64.531 52.847) (end 63.627 52.847) (width 0.25) (layer "F.Cu") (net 10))
 (segment (start 65.8622 53.3147) (end 64.9987 53.3147) (width 0.25) (layer "F.Cu") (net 10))
 (segment (start 64.9987 53.3147) (end 64.531 52.847) (width 0.25) (layer "F.Cu") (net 10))
 (segment (start 57.24 61.5) (end 54.98 61.5) (width 0.25) (layer "F.Cu") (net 6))
 (segment (start 61.62 57.12) (end 57.24 61.5) (width 0.25) (layer "F.Cu") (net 6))
 (segment (start 68.453 58.49) (end 70.41 58.49) (width 0.25) (layer "F.Cu") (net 6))
 (segment (start 70.36 58.49) (end 70.37 58.5) (width 0.25) (layer "F.Cu") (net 6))
 (segment (start 70.41 58.49) (end 70.42 58.5) (width 0.25) (layer "F.Cu") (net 6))
 (segment (start 65.659 58.4708) (end 64.3082 57.12) (width 0.25) (layer "F.Cu") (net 6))
 (segment (start 70.31 58.49) (end 70.32 58.5) (width 0.25) (layer "F.Cu") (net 6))
 (segment (start 64.3082 57.12) (end 61.62 57.12) (width 0.25) (layer "F.Cu") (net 6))
 (via (at 68.453 58.49) (size 0.6) (drill 0.3) (layers "F.Cu" "B.Cu") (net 6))
 (via (at 65.659 58.4708) (size 0.6) (drill 0.3) (layers "F.Cu" "B.Cu") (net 6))
 (segment (start 68.453 58.49) (end 65.6782 58.49) (width 0.25) (layer "B.Cu") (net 6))
 (segment (start 65.6782 58.49) (end 65.659 58.4708) (width 0.25) (layer "B.Cu") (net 6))
 (segment (start 59.7916 57.2008) (end 59.7408 57.2008) (width 0.25) (layer "F.Cu") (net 5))
 (segment (start 68.472931 59.517669) (end 70.402331 59.517669) (width 0.25) (layer "F.Cu") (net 5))
 (segment (start 68.472931 59.517669) (end 68.4906 59.5) (width 0.25) (layer "F.Cu") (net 5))
 (segment (start 70.402331 59.517669) (end 70.42 59.5) (width 0.25) (layer "F.Cu") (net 5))
 (segment (start 59.7408 57.2008) (end 56.4416 60.5) (width 0.25) (layer "F.Cu") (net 5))
 (segment (start 56.4416 60.5) (end 54.98 60.5) (width 0.25) (layer "F.Cu") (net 5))
 (segment (start 68.472931 59.517669) (end 68.455262 59.5) (width 0.25) (layer "F.Cu") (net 5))
 (segment (start 70.352331 59.517669) (end 70.37 59.5) (width 0.25) (layer "F.Cu") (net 5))
 (via (at 59.7916 57.2008) (size 0.6) (drill 0.3) (layers "F.Cu" "B.Cu") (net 5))
 (via (at 68.472931 59.517669) (size 0.6) (drill 0.3) (layers "F.Cu" "B.Cu") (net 5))
 (segment (start 61.4492 57.2008) (end 59.7916 57.2008) (width 0.25) (layer "B.Cu") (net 5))
 (segment (start 68.472931 59.517669) (end 65.791469 59.517669) (width 0.25) (layer "B.Cu") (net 5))
 (segment (start 65.791469 59.517669) (end 63.4638 57.19) (width 0.25) (layer "B.Cu") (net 5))
 (segment (start 61.46 57.19) (end 61.4492 57.2008) (width 0.25) (layer "B.Cu") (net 5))
 (segment (start 63.4638 57.19) (end 61.46 57.19) (width 0.25) (layer "B.Cu") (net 5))
 (segment (start 63.627 54.4068) (end 63.1698 54.864) (width 0.25) (layer "F.Cu") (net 9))
 (segment (start 64.5202 65.881) (end 64.5202 66.081) (width 0.25) (layer "F.Cu") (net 9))
 (segment (start 62.8402 65.941) (end 62.8452 65.936) (width 0.25) (layer "F.Cu") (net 9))
 (segment (start 63.5452 65.936) (end 64.4652 65.936) (width 0.25) (layer "F.Cu") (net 9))
 (segment (start 61.6202 65.941) (end 60.4038 65.941) (width 0.25) (layer "F.Cu") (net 9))
 (segment (start 65.6082 68.5546) (end 65.1502 68.0966) (width 0.25) (layer "F.Cu") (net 9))
 (segment (start 58.55 65.1) (end 58.55 65.5858) (width 0.25) (layer "F.Cu") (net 9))
 (segment (start 62.8452 65.936) (end 63.5452 65.936) (width 0.25) (layer "F.Cu") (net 9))
 (segment (start 61.727 52.847) (end 62.1942 52.847) (width 0.25) (layer "F.Cu") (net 9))
 (segment (start 68.5546 68.5292) (end 65.6336 68.5292) (width 0.25) (layer "F.Cu") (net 9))
 (segment (start 65.1502 66.711) (end 65.1502 67.481) (width 0.25) (layer "F.Cu") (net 9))
 (segment (start 68.4754 54.6354) (end 68.83 54.99) (width 0.25) (layer "F.Cu") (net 9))
 (segment (start 63.627 53.497) (end 64.1396 53.497) (width 0.25) (layer "F.Cu") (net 9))
 (segment (start 65.278 54.6354) (end 68.4754 54.6354) (width 0.25) (layer "F.Cu") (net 9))
 (segment (start 62.1942 52.847) (end 62.8442 53.497) (width 0.25) (layer "F.Cu") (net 9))
 (segment (start 64.5202 66.081) (end 65.1502 66.711) (width 0.25) (layer "F.Cu") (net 9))
 (segment (start 61.6202 65.941) (end 62.8402 65.941) (width 0.25) (layer "F.Cu") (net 9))
 (segment (start 59.5628 65.1) (end 58.55 65.1) (width 0.25) (layer "F.Cu") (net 9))
 (segment (start 65.6336 68.5292) (end 65.6082 68.5546) (width 0.25) (layer "F.Cu") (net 9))
 (segment (start 63.627 53.497) (end 63.627 54.4068) (width 0.25) (layer "F.Cu") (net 9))
 (segment (start 64.1396 53.497) (end 65.278 54.6354) (width 0.25) (layer "F.Cu") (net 9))
 (segment (start 69.9008 67.183) (end 68.5546 68.5292) (width 0.25) (layer "F.Cu") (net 9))
 (segment (start 60.4038 65.941) (end 59.5628 65.1) (width 0.25) (layer "F.Cu") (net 9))
 (segment (start 69.9008 63.881) (end 69.9008 67.183) (width 0.25) (layer "F.Cu") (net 9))
 (segment (start 62.8442 53.497) (end 63.627 53.497) (width 0.25) (layer "F.Cu") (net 9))
 (segment (start 65.1502 68.0966) (end 65.1502 67.481) (width 0.25) (layer "F.Cu") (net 9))
 (segment (start 64.4652 65.936) (end 64.5202 65.881) (width 0.25) (layer "F.Cu") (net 9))
 (via (at 69.9008 63.881) (size 0.6) (drill 0.3) (layers "F.Cu" "B.Cu") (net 9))
 (via (at 68.83 54.99) (size 0.6) (drill 0.3) (layers "F.Cu" "B.Cu") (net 9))
 (segment (start 69.9008 56.0832) (end 68.83 55.0124) (width 0.25) (layer "B.Cu") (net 9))
 (segment (start 68.83 55.0124) (end 68.83 54.99) (width 0.25) (layer "B.Cu") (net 9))
 (segment (start 69.9008 63.881) (end 69.9008 56.0832) (width 0.25) (layer "B.Cu") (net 9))
 (segment (start 68.426 63.981) (end 68.4276 63.9826) (width 0.25) (layer "F.Cu") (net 1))
 (segment (start 66.7952 63.981) (end 66.7952 62.8252) (width 0.25) (layer "F.Cu") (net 1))
 (segment (start 66.7952 62.8252) (end 62.7 58.73) (width 0.25) (layer "F.Cu") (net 1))
 (segment (start 62.7 58.73) (end 63.02 58.73) (width 0.25) (layer "F.Cu") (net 1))
 (segment (start 66.7952 63.981) (end 68.426 63.981) (width 0.25) (layer "F.Cu") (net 1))
 (segment (start 57.6 62.56) (end 58.89 61.27) (width 0.25) (layer "F.Cu") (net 2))
 (segment (start 57.6 63.225) (end 57.6 62.56) (width 0.25) (layer "F.Cu") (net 2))
 (segment (start 58.89 61.27) (end 62.7 61.27) (width 0.25) (layer "F.Cu") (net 2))
 (segment (start 62.0058 63.225) (end 59.5 63.225) (width 0.25) (layer "F.Cu") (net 8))
 (segment (start 59.545 63.18) (end 59.5 63.225) (width 0.25) (layer "F.Cu") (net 8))
 (segment (start 64.5202 63.981) (end 62.7618 63.981) (width 0.25) (layer "F.Cu") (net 8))
 (segment (start 62.7618 63.981) (end 62.0058 63.225) (width 0.25) (layer "F.Cu") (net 8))
 (segment (start 66.7952 67.346) (end 66.6602 67.481) (width 0.25) (layer "F.Cu") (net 7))
 (segment (start 67.7164 67.3608) (end 68.4276 67.3608) (width 0.25) (layer "F.Cu") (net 7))
 (segment (start 66.7952 65.881) (end 66.7952 67.196) (width 0.25) (layer "F.Cu") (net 7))
 (segment (start 66.5226 67.481) (end 67.5962 67.481) (width 0.25) (layer "F.Cu") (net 7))
 (segment (start 66.5226 67.481) (end 66.1702 67.481) (width 0.25) (layer "F.Cu") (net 7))
 (segment (start 66.7952 67.196) (end 66.7952 67.346) (width 0.25) (layer "F.Cu") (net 7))
 (segment (start 66.6602 67.481) (end 66.5226 67.481) (width 0.25) (layer "F.Cu") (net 7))
 (segment (start 67.5962 67.481) (end 67.7164 67.3608) (width 0.25) (layer "F.Cu") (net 7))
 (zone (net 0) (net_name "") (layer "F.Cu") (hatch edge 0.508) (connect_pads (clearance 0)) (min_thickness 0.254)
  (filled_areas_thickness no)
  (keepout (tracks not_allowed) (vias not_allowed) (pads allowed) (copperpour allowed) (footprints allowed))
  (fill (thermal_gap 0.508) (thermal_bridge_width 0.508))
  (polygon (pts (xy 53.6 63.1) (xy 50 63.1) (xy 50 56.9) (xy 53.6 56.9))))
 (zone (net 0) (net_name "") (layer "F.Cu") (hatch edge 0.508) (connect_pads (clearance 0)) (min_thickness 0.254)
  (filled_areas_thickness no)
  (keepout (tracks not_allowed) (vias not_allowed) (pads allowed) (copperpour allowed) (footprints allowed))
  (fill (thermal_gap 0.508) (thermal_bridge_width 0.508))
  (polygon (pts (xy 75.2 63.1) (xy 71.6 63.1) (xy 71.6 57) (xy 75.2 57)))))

